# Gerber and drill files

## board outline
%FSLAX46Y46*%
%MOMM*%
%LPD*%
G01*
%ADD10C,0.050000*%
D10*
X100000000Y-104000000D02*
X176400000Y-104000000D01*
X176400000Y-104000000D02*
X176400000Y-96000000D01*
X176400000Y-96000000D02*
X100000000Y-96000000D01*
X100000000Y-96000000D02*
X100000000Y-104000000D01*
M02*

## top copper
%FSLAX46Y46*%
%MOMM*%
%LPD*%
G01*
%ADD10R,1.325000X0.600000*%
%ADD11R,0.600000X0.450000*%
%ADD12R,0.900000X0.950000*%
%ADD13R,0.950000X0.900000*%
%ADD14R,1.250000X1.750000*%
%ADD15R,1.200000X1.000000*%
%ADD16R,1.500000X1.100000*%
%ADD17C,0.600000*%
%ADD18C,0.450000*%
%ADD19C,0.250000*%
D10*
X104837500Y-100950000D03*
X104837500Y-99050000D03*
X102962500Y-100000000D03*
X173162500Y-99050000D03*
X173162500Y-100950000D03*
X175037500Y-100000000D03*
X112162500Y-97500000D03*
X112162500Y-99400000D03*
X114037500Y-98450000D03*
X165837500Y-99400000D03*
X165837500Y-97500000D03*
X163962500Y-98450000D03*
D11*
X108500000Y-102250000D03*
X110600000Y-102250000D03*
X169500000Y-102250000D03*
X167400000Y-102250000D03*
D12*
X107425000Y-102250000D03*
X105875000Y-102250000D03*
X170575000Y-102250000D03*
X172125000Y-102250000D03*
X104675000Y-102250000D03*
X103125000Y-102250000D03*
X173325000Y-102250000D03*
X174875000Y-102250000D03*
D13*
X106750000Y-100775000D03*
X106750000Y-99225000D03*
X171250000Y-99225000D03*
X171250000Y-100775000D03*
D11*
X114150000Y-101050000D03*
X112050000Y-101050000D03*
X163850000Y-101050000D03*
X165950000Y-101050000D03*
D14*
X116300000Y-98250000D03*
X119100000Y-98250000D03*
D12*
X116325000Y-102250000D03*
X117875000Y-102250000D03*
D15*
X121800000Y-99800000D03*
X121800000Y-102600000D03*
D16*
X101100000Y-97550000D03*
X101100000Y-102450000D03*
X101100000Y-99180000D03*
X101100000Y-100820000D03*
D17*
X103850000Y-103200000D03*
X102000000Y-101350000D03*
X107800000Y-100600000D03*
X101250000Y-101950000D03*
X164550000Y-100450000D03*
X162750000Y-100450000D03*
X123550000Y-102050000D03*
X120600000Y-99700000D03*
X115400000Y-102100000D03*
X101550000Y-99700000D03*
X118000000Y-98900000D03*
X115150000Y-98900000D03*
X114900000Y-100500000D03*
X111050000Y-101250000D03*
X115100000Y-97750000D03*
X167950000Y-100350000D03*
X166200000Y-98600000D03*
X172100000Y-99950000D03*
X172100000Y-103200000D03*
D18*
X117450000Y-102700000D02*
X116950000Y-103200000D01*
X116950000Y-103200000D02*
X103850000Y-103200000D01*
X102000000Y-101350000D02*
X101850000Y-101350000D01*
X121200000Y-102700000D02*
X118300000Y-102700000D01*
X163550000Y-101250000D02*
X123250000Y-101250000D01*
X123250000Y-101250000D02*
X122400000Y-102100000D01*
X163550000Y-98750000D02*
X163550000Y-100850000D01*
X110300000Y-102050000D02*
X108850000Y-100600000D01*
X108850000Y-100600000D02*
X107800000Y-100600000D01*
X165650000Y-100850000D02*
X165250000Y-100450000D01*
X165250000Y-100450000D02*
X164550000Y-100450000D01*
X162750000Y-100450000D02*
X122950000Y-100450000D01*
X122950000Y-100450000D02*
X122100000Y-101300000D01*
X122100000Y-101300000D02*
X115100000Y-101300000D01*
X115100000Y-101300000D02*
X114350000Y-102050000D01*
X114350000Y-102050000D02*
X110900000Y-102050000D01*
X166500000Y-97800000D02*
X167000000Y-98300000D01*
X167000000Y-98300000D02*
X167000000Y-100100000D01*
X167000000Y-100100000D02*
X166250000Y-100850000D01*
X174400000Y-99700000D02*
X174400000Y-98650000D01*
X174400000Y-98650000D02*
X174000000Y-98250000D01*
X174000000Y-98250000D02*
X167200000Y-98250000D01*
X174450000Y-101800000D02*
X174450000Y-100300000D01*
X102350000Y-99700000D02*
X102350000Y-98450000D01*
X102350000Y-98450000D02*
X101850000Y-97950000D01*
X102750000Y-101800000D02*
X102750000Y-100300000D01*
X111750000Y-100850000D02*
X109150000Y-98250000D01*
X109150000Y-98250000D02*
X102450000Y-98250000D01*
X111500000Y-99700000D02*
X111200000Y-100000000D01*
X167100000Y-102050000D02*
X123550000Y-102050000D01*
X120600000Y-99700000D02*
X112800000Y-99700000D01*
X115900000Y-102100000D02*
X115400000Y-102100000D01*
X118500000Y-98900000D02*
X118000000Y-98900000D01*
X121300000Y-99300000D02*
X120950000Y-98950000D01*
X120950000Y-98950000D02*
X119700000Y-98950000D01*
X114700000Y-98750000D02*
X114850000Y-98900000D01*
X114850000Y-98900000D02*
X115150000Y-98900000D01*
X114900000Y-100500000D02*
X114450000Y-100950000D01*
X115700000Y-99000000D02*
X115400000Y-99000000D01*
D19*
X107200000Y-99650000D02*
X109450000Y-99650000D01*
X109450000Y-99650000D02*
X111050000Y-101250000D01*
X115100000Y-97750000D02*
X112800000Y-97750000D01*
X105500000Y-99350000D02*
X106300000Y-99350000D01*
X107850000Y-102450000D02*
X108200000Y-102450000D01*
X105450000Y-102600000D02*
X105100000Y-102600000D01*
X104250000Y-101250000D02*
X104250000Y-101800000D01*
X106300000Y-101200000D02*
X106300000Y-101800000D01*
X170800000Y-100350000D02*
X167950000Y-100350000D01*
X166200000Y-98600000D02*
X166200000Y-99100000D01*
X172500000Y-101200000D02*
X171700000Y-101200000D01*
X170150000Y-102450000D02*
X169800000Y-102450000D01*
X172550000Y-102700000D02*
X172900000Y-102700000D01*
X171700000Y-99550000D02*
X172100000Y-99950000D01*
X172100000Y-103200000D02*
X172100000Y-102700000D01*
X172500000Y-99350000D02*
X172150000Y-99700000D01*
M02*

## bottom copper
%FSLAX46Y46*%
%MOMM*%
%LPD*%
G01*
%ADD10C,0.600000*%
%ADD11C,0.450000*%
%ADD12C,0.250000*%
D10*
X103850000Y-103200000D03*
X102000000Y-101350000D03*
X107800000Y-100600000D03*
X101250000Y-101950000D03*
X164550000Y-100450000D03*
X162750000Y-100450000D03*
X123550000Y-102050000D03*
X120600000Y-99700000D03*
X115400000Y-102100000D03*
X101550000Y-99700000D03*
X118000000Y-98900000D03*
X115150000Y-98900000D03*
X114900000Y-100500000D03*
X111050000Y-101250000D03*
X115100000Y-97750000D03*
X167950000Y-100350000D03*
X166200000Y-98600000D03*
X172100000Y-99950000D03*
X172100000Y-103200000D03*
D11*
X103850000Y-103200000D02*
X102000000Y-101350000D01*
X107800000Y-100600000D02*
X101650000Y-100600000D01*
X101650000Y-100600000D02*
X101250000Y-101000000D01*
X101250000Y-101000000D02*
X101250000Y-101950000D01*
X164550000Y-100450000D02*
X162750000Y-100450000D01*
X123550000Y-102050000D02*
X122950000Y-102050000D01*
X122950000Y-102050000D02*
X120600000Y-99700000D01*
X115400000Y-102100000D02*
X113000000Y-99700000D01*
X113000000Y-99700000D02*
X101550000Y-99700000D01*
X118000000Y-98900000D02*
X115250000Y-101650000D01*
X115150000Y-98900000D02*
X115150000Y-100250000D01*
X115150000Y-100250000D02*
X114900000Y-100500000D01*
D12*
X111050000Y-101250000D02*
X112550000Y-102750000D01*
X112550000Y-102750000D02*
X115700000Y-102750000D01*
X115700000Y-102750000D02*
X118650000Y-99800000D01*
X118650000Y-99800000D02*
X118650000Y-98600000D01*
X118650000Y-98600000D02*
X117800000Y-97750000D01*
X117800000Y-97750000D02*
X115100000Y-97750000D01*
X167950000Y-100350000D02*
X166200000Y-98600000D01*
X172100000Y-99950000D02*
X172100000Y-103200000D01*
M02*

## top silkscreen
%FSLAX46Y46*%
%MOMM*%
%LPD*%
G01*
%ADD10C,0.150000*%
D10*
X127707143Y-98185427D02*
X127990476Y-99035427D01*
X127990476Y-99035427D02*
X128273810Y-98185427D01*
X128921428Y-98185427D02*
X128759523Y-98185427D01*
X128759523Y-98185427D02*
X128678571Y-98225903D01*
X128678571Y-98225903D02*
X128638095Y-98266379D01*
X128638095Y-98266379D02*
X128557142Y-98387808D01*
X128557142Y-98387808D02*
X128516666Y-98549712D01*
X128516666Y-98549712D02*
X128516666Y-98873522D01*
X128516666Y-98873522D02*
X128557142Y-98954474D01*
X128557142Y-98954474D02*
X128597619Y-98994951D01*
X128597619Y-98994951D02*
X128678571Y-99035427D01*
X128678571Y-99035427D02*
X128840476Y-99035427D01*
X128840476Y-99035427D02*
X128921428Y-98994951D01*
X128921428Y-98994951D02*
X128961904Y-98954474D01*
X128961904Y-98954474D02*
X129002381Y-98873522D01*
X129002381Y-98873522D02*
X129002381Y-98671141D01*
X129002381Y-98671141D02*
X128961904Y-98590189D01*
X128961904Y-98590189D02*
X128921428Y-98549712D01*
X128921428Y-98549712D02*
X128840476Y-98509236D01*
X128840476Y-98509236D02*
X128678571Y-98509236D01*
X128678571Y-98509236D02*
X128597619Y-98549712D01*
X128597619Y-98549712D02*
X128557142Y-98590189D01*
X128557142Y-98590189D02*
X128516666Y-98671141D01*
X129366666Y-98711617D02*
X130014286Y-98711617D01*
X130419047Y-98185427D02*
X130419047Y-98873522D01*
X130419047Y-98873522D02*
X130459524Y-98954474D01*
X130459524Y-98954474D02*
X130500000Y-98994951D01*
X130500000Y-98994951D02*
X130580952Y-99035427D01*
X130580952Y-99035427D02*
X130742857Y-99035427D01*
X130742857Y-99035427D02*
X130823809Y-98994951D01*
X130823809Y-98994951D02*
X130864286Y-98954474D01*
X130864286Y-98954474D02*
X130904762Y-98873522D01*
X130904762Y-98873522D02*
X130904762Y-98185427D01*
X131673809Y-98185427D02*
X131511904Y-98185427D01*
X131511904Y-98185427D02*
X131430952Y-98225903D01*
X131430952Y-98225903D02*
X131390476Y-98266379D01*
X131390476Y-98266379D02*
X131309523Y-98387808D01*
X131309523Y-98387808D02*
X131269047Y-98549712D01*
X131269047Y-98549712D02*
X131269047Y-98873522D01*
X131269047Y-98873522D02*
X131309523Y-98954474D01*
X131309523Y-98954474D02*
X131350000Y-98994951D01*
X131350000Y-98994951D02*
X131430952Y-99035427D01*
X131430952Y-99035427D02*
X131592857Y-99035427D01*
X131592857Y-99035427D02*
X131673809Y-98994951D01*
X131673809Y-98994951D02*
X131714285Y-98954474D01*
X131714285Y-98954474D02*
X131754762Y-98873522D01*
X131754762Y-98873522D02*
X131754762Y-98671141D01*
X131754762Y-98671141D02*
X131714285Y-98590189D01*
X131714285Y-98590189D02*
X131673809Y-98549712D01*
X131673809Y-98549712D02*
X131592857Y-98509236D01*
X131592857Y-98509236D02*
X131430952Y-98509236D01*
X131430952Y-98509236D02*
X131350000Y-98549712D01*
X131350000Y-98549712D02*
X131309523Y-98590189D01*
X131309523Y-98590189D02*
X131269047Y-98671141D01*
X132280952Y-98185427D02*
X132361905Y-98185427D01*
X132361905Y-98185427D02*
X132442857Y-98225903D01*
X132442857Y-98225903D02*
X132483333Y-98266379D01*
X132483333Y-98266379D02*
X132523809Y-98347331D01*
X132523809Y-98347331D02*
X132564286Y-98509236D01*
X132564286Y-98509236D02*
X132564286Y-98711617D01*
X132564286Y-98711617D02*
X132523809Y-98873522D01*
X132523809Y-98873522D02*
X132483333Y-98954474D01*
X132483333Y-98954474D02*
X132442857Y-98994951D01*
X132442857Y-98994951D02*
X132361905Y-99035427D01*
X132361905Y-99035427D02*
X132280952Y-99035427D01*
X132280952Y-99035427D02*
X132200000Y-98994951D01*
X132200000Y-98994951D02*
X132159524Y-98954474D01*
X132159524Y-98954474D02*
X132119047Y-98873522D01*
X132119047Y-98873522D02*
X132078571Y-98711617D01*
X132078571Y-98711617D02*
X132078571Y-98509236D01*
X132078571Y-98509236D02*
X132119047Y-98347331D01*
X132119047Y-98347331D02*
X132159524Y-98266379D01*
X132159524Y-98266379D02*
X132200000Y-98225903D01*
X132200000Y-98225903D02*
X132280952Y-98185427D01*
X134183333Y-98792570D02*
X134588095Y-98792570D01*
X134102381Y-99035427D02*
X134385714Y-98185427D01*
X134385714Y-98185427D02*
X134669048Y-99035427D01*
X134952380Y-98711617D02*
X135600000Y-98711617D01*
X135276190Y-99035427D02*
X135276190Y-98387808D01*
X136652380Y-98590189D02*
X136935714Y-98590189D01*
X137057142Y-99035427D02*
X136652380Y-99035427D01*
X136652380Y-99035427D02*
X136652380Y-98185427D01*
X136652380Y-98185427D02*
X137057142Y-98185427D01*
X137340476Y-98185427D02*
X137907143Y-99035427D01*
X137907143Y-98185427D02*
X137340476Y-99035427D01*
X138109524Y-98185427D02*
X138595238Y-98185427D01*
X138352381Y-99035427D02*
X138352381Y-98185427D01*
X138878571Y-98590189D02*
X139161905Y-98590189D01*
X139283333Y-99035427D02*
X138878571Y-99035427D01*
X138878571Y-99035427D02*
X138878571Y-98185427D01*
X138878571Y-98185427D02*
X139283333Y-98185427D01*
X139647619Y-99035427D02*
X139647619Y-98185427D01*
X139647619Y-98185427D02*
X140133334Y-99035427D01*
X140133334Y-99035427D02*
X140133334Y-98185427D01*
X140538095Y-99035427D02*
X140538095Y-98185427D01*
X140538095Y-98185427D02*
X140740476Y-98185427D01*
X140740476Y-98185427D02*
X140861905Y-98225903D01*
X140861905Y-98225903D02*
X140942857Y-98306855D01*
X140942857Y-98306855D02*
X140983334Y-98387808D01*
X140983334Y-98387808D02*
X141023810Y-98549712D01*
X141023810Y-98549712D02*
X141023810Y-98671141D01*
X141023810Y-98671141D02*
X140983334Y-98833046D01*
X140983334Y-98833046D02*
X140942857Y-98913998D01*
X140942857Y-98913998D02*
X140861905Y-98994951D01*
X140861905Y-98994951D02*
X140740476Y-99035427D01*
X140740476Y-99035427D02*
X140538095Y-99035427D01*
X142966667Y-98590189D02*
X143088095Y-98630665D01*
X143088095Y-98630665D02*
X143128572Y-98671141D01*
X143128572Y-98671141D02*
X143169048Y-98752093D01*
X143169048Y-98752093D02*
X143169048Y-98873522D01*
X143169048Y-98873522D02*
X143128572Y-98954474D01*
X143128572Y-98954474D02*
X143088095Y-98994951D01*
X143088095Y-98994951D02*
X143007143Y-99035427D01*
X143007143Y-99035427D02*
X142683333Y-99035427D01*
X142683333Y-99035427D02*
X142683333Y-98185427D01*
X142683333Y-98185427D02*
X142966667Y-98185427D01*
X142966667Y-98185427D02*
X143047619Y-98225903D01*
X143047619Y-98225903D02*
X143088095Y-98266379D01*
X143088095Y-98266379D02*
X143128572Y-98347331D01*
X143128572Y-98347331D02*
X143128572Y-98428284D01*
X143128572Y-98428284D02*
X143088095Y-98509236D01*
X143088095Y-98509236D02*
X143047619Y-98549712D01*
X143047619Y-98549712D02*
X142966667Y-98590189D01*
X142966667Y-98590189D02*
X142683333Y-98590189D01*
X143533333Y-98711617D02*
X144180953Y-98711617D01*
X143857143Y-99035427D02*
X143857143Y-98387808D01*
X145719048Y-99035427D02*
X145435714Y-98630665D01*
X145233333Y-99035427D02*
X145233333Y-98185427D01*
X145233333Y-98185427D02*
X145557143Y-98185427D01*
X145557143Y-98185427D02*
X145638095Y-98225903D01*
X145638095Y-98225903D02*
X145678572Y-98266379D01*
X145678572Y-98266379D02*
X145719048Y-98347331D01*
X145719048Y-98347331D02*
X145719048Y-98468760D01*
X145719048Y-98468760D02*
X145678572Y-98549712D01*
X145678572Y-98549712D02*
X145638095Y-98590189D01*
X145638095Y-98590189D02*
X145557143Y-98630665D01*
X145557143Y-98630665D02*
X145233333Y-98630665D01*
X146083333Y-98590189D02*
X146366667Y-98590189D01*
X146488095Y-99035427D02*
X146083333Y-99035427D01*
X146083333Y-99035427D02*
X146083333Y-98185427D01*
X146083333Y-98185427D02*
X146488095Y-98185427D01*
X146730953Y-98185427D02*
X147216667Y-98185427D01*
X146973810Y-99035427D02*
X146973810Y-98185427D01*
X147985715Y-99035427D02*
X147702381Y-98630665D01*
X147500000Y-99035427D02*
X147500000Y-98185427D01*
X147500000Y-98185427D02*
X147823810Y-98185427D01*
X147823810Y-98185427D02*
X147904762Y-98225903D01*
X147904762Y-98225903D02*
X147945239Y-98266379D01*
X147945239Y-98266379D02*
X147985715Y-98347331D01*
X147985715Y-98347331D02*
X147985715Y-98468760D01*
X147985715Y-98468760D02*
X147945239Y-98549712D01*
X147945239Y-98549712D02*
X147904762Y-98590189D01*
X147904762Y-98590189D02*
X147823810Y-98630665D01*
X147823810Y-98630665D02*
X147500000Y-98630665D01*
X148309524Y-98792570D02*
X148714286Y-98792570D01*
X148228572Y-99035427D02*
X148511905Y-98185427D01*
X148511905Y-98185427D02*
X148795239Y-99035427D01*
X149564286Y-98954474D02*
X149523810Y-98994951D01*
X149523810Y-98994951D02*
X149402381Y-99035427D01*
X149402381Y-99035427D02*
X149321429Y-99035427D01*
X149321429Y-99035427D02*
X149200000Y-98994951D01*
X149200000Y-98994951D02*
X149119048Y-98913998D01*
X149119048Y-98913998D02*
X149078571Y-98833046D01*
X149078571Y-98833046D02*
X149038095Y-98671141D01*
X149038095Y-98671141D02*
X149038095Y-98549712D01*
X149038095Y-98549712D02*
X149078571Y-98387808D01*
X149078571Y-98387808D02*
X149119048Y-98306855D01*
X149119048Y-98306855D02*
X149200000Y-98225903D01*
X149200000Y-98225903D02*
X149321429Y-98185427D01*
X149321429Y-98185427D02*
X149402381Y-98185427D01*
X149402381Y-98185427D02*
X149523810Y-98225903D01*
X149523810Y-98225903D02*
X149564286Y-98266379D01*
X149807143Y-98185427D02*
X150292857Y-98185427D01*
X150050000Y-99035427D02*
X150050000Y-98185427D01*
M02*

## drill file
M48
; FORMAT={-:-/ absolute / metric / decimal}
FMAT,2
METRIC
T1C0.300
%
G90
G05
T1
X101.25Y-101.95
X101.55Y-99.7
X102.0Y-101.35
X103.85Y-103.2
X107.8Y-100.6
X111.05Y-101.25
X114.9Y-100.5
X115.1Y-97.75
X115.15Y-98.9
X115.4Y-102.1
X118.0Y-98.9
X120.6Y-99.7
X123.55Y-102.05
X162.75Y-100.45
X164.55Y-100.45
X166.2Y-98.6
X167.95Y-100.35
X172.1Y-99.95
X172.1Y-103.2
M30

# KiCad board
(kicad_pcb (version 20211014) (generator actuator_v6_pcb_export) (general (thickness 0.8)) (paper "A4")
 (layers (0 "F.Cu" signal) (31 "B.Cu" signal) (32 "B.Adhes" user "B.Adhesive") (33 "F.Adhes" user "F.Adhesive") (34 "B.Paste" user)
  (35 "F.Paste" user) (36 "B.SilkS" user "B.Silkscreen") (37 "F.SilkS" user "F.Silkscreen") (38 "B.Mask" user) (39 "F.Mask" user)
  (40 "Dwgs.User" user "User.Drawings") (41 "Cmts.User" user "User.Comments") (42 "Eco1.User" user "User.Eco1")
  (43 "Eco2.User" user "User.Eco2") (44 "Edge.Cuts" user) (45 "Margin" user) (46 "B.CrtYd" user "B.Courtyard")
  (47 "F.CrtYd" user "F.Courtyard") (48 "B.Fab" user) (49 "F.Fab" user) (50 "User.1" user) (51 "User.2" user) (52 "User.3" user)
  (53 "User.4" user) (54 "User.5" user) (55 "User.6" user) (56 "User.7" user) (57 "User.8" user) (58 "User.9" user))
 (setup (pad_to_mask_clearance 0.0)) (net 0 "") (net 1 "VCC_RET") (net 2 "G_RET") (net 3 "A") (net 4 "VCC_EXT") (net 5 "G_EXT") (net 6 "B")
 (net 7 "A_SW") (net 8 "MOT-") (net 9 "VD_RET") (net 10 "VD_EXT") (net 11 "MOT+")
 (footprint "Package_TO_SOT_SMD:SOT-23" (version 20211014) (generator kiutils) (layer "F.Cu") (at 103.9 100.0 180)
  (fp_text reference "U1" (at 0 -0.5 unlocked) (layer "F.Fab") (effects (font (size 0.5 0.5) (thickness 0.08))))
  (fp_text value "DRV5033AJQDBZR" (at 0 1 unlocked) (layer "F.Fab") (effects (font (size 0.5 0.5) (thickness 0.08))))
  (pad "1" smd rect (at -0.9375 -0.95 180) (size 1.325 0.6) (layers "F.Cu" "F.Mask" "F.Paste") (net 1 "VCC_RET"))
  (pad "2" smd rect (at -0.9375 0.95 180) (size 1.325 0.6) (layers "F.Cu" "F.Mask" "F.Paste") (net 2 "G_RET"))
  (pad "3" smd rect (at 0.9375 0.0 180) (size 1.325 0.6) (layers "F.Cu" "F.Mask" "F.Paste") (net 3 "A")))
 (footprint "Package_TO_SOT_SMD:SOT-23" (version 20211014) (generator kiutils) (layer "F.Cu") (at 174.1 100.0)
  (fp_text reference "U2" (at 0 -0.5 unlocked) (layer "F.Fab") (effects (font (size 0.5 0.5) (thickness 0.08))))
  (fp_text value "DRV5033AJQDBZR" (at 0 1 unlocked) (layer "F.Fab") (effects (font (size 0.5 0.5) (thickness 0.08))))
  (pad "1" smd rect (at -0.9375 -0.95) (size 1.325 0.6) (layers "F.Cu" "F.Mask" "F.Paste") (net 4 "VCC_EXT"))
  (pad "2" smd rect (at -0.9375 0.95) (size 1.325 0.6) (layers "F.Cu" "F.Mask" "F.Paste") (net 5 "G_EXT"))
  (pad "3" smd rect (at 0.9375 0.0) (size 1.325 0.6) (layers "F.Cu" "F.Mask" "F.Paste") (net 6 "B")))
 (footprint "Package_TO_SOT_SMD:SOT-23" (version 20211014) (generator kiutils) (layer "F.Cu") (at 113.1 98.45)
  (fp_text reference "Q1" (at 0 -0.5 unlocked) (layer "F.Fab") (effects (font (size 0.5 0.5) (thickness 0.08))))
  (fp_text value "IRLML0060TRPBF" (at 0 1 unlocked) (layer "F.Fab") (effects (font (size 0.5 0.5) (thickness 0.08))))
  (pad "1" smd rect (at -0.9375 -0.95) (size 1.325 0.6) (layers "F.Cu" "F.Mask" "F.Paste") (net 2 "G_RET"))
  (pad "2" smd rect (at -0.9375 0.95) (size 1.325 0.6) (layers "F.Cu" "F.Mask" "F.Paste") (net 3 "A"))
  (pad "3" smd rect (at 0.9375 0.0) (size 1.325 0.6) (layers "F.Cu" "F.Mask" "F.Paste") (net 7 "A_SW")))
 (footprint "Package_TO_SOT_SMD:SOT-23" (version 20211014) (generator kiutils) (layer "F.Cu") (at 164.9 98.45 180)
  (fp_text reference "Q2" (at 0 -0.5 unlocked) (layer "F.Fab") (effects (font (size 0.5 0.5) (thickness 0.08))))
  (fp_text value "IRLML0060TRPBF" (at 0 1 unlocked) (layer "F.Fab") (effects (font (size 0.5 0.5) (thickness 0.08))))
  (pad "1" smd rect (at -0.9375 -0.95 180) (size 1.325 0.6) (layers "F.Cu" "F.Mask" "F.Paste") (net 5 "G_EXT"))
  (pad "2" smd rect (at -0.9375 0.95 180) (size 1.325 0.6) (layers "F.Cu" "F.Mask" "F.Paste") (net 6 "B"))
  (pad "3" smd rect (at 0.9375 0.0 180) (size 1.325 0.6) (layers "F.Cu" "F.Mask" "F.Paste") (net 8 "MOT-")))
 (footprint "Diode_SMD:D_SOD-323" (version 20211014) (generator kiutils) (layer "F.Cu") (at 109.55 102.25)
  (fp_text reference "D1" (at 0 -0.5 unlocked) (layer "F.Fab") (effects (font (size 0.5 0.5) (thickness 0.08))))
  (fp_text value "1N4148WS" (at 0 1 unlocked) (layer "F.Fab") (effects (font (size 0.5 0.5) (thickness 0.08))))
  (pad "1" smd rect (at -1.05 0.0) (size 0.6 0.45) (layers "F.Cu" "F.Mask" "F.Paste") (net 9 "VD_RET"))
  (pad "2" smd rect (at 1.05 0.0) (size 0.6 0.45) (layers "F.Cu" "F.Mask" "F.Paste") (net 6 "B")))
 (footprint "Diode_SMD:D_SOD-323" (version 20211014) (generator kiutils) (layer "F.Cu") (at 168.45 102.25 180)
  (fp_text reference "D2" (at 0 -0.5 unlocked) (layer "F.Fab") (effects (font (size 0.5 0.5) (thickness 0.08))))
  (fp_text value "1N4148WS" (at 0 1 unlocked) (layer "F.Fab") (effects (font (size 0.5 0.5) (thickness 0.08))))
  (pad "1" smd rect (at -1.05 0.0 180) (size 0.6 0.45) (layers "F.Cu" "F.Mask" "F.Paste") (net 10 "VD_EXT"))
  (pad "2" smd rect (at 1.05 0.0 180) (size 0.6 0.45) (layers "F.Cu" "F.Mask" "F.Paste") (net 3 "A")))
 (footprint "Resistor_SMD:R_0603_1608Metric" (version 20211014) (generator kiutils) (layer "F.Cu") (at 106.65 102.25 180)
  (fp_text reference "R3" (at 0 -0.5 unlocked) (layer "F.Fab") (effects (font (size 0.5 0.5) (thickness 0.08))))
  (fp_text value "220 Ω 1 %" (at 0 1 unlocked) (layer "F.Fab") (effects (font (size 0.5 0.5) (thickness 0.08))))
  (pad "1" smd rect (at -0.775 0.0 180) (size 0.9 0.95) (layers "F.Cu" "F.Mask" "F.Paste") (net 9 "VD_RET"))
  (pad "2" smd rect (at 0.775 0.0 180) (size 0.9 0.95) (layers "F.Cu" "F.Mask" "F.Paste") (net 1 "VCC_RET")))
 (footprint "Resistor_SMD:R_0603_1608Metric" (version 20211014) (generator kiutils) (layer "F.Cu") (at 171.35 102.25)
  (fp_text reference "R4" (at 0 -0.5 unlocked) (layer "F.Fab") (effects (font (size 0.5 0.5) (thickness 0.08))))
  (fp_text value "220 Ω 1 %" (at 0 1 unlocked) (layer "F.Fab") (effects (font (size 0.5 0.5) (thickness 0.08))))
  (pad "1" smd rect (at -0.775 0.0) (size 0.9 0.95) (layers "F.Cu" "F.Mask" "F.Paste") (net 10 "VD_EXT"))
  (pad "2" smd rect (at 0.775 0.0) (size 0.9 0.95) (layers "F.Cu" "F.Mask" "F.Paste") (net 4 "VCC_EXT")))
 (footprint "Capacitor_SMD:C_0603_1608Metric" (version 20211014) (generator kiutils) (layer "F.Cu") (at 103.9 102.25 180)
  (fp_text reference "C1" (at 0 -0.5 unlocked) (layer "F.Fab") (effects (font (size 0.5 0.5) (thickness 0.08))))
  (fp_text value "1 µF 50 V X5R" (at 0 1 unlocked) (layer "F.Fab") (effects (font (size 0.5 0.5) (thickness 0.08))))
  (pad "1" smd rect (at -0.775 0.0 180) (size 0.9 0.95) (layers "F.Cu" "F.Mask" "F.Paste") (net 1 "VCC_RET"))
  (pad "2" smd rect (at 0.775 0.0 180) (size 0.9 0.95) (layers "F.Cu" "F.Mask" "F.Paste") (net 3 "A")))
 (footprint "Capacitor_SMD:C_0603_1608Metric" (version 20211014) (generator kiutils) (layer "F.Cu") (at 174.1 102.25)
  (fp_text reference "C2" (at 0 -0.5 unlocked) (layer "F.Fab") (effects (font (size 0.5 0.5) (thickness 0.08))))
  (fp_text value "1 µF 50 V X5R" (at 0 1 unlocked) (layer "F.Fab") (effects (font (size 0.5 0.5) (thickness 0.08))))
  (pad "1" smd rect (at -0.775 0.0) (size 0.9 0.95) (layers "F.Cu" "F.Mask" "F.Paste") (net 4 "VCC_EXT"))
  (pad "2" smd rect (at 0.775 0.0) (size 0.9 0.95) (layers "F.Cu" "F.Mask" "F.Paste") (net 6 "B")))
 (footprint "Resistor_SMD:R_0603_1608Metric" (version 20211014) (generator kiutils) (layer "F.Cu") (at 106.75 100.0 90)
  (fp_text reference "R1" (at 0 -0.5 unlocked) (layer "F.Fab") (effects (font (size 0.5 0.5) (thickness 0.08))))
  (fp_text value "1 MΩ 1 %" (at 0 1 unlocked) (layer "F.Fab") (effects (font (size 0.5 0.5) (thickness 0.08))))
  (pad "1" smd rect (at -0.775 0.0 90) (size 0.9 0.95) (layers "F.Cu" "F.Mask" "F.Paste") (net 1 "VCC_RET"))
  (pad "2" smd rect (at 0.775 0.0 90) (size 0.9 0.95) (layers "F.Cu" "F.Mask" "F.Paste") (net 2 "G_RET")))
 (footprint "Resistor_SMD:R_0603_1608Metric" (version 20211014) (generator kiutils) (layer "F.Cu") (at 171.25 100.0 270)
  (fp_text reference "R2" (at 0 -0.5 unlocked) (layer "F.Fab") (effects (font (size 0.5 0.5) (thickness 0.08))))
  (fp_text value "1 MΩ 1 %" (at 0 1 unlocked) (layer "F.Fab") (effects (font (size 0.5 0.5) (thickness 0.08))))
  (pad "1" smd rect (at -0.775 0.0 270) (size 0.9 0.95) (layers "F.Cu" "F.Mask" "F.Paste") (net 4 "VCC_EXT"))
  (pad "2" smd rect (at 0.775 0.0 270) (size 0.9 0.95) (layers "F.Cu" "F.Mask" "F.Paste") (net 5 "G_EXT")))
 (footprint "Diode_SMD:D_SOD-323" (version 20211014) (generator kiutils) (layer "F.Cu") (at 113.1 101.05 180)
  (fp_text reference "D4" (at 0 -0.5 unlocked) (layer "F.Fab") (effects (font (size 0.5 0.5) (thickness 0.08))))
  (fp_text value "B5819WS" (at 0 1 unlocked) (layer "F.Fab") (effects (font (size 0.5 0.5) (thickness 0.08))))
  (pad "1" smd rect (at -1.05 0.0 180) (size 0.6 0.45) (layers "F.Cu" "F.Mask" "F.Paste") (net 7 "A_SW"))
  (pad "2" smd rect (at 1.05 0.0 180) (size 0.6 0.45) (layers "F.Cu" "F.Mask" "F.Paste") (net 3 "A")))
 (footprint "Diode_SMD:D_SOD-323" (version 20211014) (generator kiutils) (layer "F.Cu") (at 164.9 101.05)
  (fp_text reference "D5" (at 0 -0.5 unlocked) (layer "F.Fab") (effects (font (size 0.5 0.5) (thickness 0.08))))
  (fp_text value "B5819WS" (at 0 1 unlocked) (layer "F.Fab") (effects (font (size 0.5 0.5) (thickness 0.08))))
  (pad "1" smd rect (at -1.05 0.0) (size 0.6 0.45) (layers "F.Cu" "F.Mask" "F.Paste") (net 8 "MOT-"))
  (pad "2" smd rect (at 1.05 0.0) (size 0.6 0.45) (layers "F.Cu" "F.Mask" "F.Paste") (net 6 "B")))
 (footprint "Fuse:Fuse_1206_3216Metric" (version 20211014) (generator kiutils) (layer "F.Cu") (at 117.7 98.25)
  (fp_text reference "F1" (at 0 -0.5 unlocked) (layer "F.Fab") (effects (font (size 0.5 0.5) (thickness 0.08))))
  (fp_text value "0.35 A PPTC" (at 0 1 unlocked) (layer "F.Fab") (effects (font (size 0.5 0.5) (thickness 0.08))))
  (pad "1" smd rect (at -1.4 0.0) (size 1.25 1.75) (layers "F.Cu" "F.Mask" "F.Paste") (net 7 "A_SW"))
  (pad "2" smd rect (at 1.4 0.0) (size 1.25 1.75) (layers "F.Cu" "F.Mask" "F.Paste") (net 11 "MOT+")))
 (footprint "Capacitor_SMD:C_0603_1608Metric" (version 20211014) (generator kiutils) (layer "F.Cu") (at 117.1 102.25)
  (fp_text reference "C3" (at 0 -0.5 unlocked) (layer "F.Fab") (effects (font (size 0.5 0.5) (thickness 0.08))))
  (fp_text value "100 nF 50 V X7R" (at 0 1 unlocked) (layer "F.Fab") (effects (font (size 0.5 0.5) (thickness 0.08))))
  (pad "1" smd rect (at -0.775 0.0) (size 0.9 0.95) (layers "F.Cu" "F.Mask" "F.Paste") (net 11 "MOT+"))
  (pad "2" smd rect (at 0.775 0.0) (size 0.9 0.95) (layers "F.Cu" "F.Mask" "F.Paste") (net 8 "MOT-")))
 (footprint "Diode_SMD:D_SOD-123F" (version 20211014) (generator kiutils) (layer "F.Cu") (at 121.8 101.2 270)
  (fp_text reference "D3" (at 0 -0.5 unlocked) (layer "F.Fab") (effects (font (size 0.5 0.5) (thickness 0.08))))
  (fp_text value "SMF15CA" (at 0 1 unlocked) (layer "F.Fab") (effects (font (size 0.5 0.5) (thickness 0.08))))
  (pad "1" smd rect (at -1.4 0.0 270) (size 1.0 1.2) (layers "F.Cu" "F.Mask" "F.Paste") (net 11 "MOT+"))
  (pad "2" smd rect (at 1.4 0.0 270) (size 1.0 1.2) (layers "F.Cu" "F.Mask" "F.Paste") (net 8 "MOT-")))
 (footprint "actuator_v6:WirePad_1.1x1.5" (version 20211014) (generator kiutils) (layer "F.Cu") (at 101.1 97.55)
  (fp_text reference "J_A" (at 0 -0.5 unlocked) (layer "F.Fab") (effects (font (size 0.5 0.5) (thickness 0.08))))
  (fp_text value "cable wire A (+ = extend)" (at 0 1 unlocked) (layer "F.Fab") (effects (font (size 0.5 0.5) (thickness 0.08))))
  (pad "1" smd rect (at 0.0 0.0) (size 1.5 1.1) (layers "F.Cu" "F.Mask") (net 3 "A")))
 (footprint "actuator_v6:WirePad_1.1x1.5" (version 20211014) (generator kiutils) (layer "F.Cu") (at 101.1 102.45)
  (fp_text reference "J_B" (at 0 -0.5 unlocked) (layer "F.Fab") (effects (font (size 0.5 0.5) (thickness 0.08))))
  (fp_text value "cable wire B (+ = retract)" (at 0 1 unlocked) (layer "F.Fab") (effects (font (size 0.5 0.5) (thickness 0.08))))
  (pad "1" smd rect (at 0.0 0.0) (size 1.5 1.1) (layers "F.Cu" "F.Mask") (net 6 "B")))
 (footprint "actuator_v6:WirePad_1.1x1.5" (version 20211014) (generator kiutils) (layer "F.Cu") (at 101.1 99.18)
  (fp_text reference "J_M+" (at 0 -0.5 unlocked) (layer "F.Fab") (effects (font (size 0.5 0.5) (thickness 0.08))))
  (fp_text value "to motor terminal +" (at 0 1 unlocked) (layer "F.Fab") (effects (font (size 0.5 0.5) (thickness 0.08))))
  (pad "1" smd rect (at 0.0 0.0) (size 1.5 1.1) (layers "F.Cu" "F.Mask") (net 11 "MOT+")))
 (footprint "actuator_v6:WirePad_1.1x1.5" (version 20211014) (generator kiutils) (layer "F.Cu") (at 101.1 100.82)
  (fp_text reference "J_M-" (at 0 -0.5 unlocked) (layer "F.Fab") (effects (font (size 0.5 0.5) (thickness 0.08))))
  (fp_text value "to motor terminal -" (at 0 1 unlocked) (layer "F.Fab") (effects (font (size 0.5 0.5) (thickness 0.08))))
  (pad "1" smd rect (at 0.0 0.0) (size 1.5 1.1) (layers "F.Cu" "F.Mask") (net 8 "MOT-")))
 (gr_line (start 100.0 104.0) (end 176.4 104.0) (layer "Edge.Cuts") (width 0.05))
 (gr_line (start 176.4 104.0) (end 176.4 96.0) (layer "Edge.Cuts") (width 0.05))
 (gr_line (start 176.4 96.0) (end 100.0 96.0) (layer "Edge.Cuts") (width 0.05))
 (gr_line (start 100.0 96.0) (end 100.0 104.0) (layer "Edge.Cuts") (width 0.05))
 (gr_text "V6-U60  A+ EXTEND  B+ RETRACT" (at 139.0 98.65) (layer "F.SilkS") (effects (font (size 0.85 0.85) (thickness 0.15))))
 (segment (start 117.45 102.7) (end 116.95 103.2) (width 0.45) (layer "F.Cu") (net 8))
 (segment (start 116.95 103.2) (end 103.85 103.2) (width 0.45) (layer "F.Cu") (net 8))
 (segment (start 103.85 103.2) (end 102.0 101.35) (width 0.45) (layer "B.Cu") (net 8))
 (segment (start 102.0 101.35) (end 101.85 101.35) (width 0.45) (layer "F.Cu") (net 8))
 (segment (start 121.2 102.7) (end 118.3 102.7) (width 0.45) (layer "F.Cu") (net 8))
 (segment (start 163.55 101.25) (end 123.25 101.25) (width 0.45) (layer "F.Cu") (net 8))
 (segment (start 123.25 101.25) (end 122.4 102.1) (width 0.45) (layer "F.Cu") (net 8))
 (segment (start 163.55 98.75) (end 163.55 100.85) (width 0.45) (layer "F.Cu") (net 8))
 (segment (start 110.3 102.05) (end 108.85 100.6) (width 0.45) (layer "F.Cu") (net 6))
 (segment (start 108.85 100.6) (end 107.8 100.6) (width 0.45) (layer "F.Cu") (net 6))
 (segment (start 107.8 100.6) (end 101.65 100.6) (width 0.45) (layer "B.Cu") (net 6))
 (segment (start 101.65 100.6) (end 101.25 101.0) (width 0.45) (layer "B.Cu") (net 6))
 (segment (start 101.25 101.0) (end 101.25 101.95) (width 0.45) (layer "B.Cu") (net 6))
 (segment (start 165.65 100.85) (end 165.25 100.45) (width 0.45) (layer "F.Cu") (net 6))
 (segment (start 165.25 100.45) (end 164.55 100.45) (width 0.45) (layer "F.Cu") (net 6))
 (segment (start 164.55 100.45) (end 162.75 100.45) (width 0.45) (layer "B.Cu") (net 6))
 (segment (start 162.75 100.45) (end 122.95 100.45) (width 0.45) (layer "F.Cu") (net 6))
 (segment (start 122.95 100.45) (end 122.1 101.3) (width 0.45) (layer "F.Cu") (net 6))
 (segment (start 122.1 101.3) (end 115.1 101.3) (width 0.45) (layer "F.Cu") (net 6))
 (segment (start 115.1 101.3) (end 114.35 102.05) (width 0.45) (layer "F.Cu") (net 6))
 (segment (start 114.35 102.05) (end 110.9 102.05) (width 0.45) (layer "F.Cu") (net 6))
 (segment (start 166.5 97.8) (end 167.0 98.3) (width 0.45) (layer "F.Cu") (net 6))
 (segment (start 167.0 98.3) (end 167.0 100.1) (width 0.45) (layer "F.Cu") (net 6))
 (segment (start 167.0 100.1) (end 166.25 100.85) (width 0.45) (layer "F.Cu") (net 6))
 (segment (start 174.4 99.7) (end 174.4 98.65) (width 0.45) (layer "F.Cu") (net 6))
 (segment (start 174.4 98.65) (end 174.0 98.25) (width 0.45) (layer "F.Cu") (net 6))
 (segment (start 174.0 98.25) (end 167.2 98.25) (width 0.45) (layer "F.Cu") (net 6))
 (segment (start 174.45 101.8) (end 174.45 100.3) (width 0.45) (layer "F.Cu") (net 6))
 (segment (start 102.35 99.7) (end 102.35 98.45) (width 0.45) (layer "F.Cu") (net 3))
 (segment (start 102.35 98.45) (end 101.85 97.95) (width 0.45) (layer "F.Cu") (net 3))
 (segment (start 102.75 101.8) (end 102.75 100.3) (width 0.45) (layer "F.Cu") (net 3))
 (segment (start 111.75 100.85) (end 109.15 98.25) (width 0.45) (layer "F.Cu") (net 3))
 (segment (start 109.15 98.25) (end 102.45 98.25) (width 0.45) (layer "F.Cu") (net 3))
 (segment (start 111.5 99.7) (end 111.2 100.0) (width 0.45) (layer "F.Cu") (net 3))
 (segment (start 167.1 102.05) (end 123.55 102.05) (width 0.45) (layer "F.Cu") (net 3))
 (segment (start 123.55 102.05) (end 122.95 102.05) (width 0.45) (layer "B.Cu") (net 3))
 (segment (start 122.95 102.05) (end 120.6 99.7) (width 0.45) (layer "B.Cu") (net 3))
 (segment (start 120.6 99.7) (end 112.8 99.7) (width 0.45) (layer "F.Cu") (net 3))
 (segment (start 115.9 102.1) (end 115.4 102.1) (width 0.45) (layer "F.Cu") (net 11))
 (segment (start 115.4 102.1) (end 113.0 99.7) (width 0.45) (layer "B.Cu") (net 11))
 (segment (start 113.0 99.7) (end 101.55 99.7) (width 0.45) (layer "B.Cu") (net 11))
 (segment (start 118.5 98.9) (end 118.0 98.9) (width 0.45) (layer "F.Cu") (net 11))
 (segment (start 118.0 98.9) (end 115.25 101.65) (width 0.45) (layer "B.Cu") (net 11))
 (segment (start 121.3 99.3) (end 120.95 98.95) (width 0.45) (layer "F.Cu") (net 11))
 (segment (start 120.95 98.95) (end 119.7 98.95) (width 0.45) (layer "F.Cu") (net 11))
 (segment (start 114.7 98.75) (end 114.85 98.9) (width 0.45) (layer "F.Cu") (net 7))
 (segment (start 114.85 98.9) (end 115.15 98.9) (width 0.45) (layer "F.Cu") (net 7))
 (segment (start 115.15 98.9) (end 115.15 100.25) (width 0.45) (layer "B.Cu") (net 7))
 (segment (start 115.15 100.25) (end 114.9 100.5) (width 0.45) (layer "B.Cu") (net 7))
 (segment (start 114.9 100.5) (end 114.45 100.95) (width 0.45) (layer "F.Cu") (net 7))
 (segment (start 115.7 99.0) (end 115.4 99.0) (width 0.45) (layer "F.Cu") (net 7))
 (segment (start 107.2 99.65) (end 109.45 99.65) (width 0.25) (layer "F.Cu") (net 2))
 (segment (start 109.45 99.65) (end 111.05 101.25) (width 0.25) (layer "F.Cu") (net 2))
 (segment (start 111.05 101.25) (end 112.55 102.75) (width 0.25) (layer "B.Cu") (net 2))
 (segment (start 112.55 102.75) (end 115.7 102.75) (width 0.25) (layer "B.Cu") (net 2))
 (segment (start 115.7 102.75) (end 118.65 99.8) (width 0.25) (layer "B.Cu") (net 2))
 (segment (start 118.65 99.8) (end 118.65 98.6) (width 0.25) (layer "B.Cu") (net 2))
 (segment (start 118.65 98.6) (end 117.8 97.75) (width 0.25) (layer "B.Cu") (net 2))
 (segment (start 117.8 97.75) (end 115.1 97.75) (width 0.25) (layer "B.Cu") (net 2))
 (segment (start 115.1 97.75) (end 112.8 97.75) (width 0.25) (layer "F.Cu") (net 2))
 (segment (start 105.5 99.35) (end 106.3 99.35) (width 0.25) (layer "F.Cu") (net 2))
 (segment (start 107.85 102.45) (end 108.2 102.45) (width 0.25) (layer "F.Cu") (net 9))
 (segment (start 105.45 102.6) (end 105.1 102.6) (width 0.25) (layer "F.Cu") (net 1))
 (segment (start 104.25 101.25) (end 104.25 101.8) (width 0.25) (layer "F.Cu") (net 1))
 (segment (start 106.3 101.2) (end 106.3 101.8) (width 0.25) (layer "F.Cu") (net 1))
 (segment (start 170.8 100.35) (end 167.95 100.35) (width 0.25) (layer "F.Cu") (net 5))
 (segment (start 167.95 100.35) (end 166.2 98.6) (width 0.25) (layer "B.Cu") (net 5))
 (segment (start 166.2 98.6) (end 166.2 99.1) (width 0.25) (layer "F.Cu") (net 5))
 (segment (start 172.5 101.2) (end 171.7 101.2) (width 0.25) (layer "F.Cu") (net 5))
 (segment (start 170.15 102.45) (end 169.8 102.45) (width 0.25) (layer "F.Cu") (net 10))
 (segment (start 172.55 102.7) (end 172.9 102.7) (width 0.25) (layer "F.Cu") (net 4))
 (segment (start 171.7 99.55) (end 172.1 99.95) (width 0.25) (layer "F.Cu") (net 4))
 (segment (start 172.1 99.95) (end 172.1 103.2) (width 0.25) (layer "B.Cu") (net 4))
 (segment (start 172.1 103.2) (end 172.1 102.7) (width 0.25) (layer "F.Cu") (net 4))
 (segment (start 172.5 99.35) (end 172.15 99.7) (width 0.25) (layer "F.Cu") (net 4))
 (via (at 103.85 103.2) (size 0.6) (drill 0.3) (layers "F.Cu" "B.Cu") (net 8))
 (via (at 102.0 101.35) (size 0.6) (drill 0.3) (layers "F.Cu" "B.Cu") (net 8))
 (via (at 107.8 100.6) (size 0.6) (drill 0.3) (layers "F.Cu" "B.Cu") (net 6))
 (via (at 101.25 101.95) (size 0.6) (drill 0.3) (layers "F.Cu" "B.Cu") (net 6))
 (via (at 164.55 100.45) (size 0.6) (drill 0.3) (layers "F.Cu" "B.Cu") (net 6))
 (via (at 162.75 100.45) (size 0.6) (drill 0.3) (layers "F.Cu" "B.Cu") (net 6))
 (via (at 123.55 102.05) (size 0.6) (drill 0.3) (layers "F.Cu" "B.Cu") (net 3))
 (via (at 120.6 99.7) (size 0.6) (drill 0.3) (layers "F.Cu" "B.Cu") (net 3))
 (via (at 115.4 102.1) (size 0.6) (drill 0.3) (layers "F.Cu" "B.Cu") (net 11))
 (via (at 101.55 99.7) (size 0.6) (drill 0.3) (layers "F.Cu" "B.Cu") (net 11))
 (via (at 118.0 98.9) (size 0.6) (drill 0.3) (layers "F.Cu" "B.Cu") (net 11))
 (via (at 115.15 98.9) (size 0.6) (drill 0.3) (layers "F.Cu" "B.Cu") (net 7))
 (via (at 114.9 100.5) (size 0.6) (drill 0.3) (layers "F.Cu" "B.Cu") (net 7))
 (via (at 111.05 101.25) (size 0.6) (drill 0.3) (layers "F.Cu" "B.Cu") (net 2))
 (via (at 115.1 97.75) (size 0.6) (drill 0.3) (layers "F.Cu" "B.Cu") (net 2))
 (via (at 167.95 100.35) (size 0.6) (drill 0.3) (layers "F.Cu" "B.Cu") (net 5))
 (via (at 166.2 98.6) (size 0.6) (drill 0.3) (layers "F.Cu" "B.Cu") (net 5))
 (via (at 172.1 99.95) (size 0.6) (drill 0.3) (layers "F.Cu" "B.Cu") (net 4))
 (via (at 172.1 103.2) (size 0.6) (drill 0.3) (layers "F.Cu" "B.Cu") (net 4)))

